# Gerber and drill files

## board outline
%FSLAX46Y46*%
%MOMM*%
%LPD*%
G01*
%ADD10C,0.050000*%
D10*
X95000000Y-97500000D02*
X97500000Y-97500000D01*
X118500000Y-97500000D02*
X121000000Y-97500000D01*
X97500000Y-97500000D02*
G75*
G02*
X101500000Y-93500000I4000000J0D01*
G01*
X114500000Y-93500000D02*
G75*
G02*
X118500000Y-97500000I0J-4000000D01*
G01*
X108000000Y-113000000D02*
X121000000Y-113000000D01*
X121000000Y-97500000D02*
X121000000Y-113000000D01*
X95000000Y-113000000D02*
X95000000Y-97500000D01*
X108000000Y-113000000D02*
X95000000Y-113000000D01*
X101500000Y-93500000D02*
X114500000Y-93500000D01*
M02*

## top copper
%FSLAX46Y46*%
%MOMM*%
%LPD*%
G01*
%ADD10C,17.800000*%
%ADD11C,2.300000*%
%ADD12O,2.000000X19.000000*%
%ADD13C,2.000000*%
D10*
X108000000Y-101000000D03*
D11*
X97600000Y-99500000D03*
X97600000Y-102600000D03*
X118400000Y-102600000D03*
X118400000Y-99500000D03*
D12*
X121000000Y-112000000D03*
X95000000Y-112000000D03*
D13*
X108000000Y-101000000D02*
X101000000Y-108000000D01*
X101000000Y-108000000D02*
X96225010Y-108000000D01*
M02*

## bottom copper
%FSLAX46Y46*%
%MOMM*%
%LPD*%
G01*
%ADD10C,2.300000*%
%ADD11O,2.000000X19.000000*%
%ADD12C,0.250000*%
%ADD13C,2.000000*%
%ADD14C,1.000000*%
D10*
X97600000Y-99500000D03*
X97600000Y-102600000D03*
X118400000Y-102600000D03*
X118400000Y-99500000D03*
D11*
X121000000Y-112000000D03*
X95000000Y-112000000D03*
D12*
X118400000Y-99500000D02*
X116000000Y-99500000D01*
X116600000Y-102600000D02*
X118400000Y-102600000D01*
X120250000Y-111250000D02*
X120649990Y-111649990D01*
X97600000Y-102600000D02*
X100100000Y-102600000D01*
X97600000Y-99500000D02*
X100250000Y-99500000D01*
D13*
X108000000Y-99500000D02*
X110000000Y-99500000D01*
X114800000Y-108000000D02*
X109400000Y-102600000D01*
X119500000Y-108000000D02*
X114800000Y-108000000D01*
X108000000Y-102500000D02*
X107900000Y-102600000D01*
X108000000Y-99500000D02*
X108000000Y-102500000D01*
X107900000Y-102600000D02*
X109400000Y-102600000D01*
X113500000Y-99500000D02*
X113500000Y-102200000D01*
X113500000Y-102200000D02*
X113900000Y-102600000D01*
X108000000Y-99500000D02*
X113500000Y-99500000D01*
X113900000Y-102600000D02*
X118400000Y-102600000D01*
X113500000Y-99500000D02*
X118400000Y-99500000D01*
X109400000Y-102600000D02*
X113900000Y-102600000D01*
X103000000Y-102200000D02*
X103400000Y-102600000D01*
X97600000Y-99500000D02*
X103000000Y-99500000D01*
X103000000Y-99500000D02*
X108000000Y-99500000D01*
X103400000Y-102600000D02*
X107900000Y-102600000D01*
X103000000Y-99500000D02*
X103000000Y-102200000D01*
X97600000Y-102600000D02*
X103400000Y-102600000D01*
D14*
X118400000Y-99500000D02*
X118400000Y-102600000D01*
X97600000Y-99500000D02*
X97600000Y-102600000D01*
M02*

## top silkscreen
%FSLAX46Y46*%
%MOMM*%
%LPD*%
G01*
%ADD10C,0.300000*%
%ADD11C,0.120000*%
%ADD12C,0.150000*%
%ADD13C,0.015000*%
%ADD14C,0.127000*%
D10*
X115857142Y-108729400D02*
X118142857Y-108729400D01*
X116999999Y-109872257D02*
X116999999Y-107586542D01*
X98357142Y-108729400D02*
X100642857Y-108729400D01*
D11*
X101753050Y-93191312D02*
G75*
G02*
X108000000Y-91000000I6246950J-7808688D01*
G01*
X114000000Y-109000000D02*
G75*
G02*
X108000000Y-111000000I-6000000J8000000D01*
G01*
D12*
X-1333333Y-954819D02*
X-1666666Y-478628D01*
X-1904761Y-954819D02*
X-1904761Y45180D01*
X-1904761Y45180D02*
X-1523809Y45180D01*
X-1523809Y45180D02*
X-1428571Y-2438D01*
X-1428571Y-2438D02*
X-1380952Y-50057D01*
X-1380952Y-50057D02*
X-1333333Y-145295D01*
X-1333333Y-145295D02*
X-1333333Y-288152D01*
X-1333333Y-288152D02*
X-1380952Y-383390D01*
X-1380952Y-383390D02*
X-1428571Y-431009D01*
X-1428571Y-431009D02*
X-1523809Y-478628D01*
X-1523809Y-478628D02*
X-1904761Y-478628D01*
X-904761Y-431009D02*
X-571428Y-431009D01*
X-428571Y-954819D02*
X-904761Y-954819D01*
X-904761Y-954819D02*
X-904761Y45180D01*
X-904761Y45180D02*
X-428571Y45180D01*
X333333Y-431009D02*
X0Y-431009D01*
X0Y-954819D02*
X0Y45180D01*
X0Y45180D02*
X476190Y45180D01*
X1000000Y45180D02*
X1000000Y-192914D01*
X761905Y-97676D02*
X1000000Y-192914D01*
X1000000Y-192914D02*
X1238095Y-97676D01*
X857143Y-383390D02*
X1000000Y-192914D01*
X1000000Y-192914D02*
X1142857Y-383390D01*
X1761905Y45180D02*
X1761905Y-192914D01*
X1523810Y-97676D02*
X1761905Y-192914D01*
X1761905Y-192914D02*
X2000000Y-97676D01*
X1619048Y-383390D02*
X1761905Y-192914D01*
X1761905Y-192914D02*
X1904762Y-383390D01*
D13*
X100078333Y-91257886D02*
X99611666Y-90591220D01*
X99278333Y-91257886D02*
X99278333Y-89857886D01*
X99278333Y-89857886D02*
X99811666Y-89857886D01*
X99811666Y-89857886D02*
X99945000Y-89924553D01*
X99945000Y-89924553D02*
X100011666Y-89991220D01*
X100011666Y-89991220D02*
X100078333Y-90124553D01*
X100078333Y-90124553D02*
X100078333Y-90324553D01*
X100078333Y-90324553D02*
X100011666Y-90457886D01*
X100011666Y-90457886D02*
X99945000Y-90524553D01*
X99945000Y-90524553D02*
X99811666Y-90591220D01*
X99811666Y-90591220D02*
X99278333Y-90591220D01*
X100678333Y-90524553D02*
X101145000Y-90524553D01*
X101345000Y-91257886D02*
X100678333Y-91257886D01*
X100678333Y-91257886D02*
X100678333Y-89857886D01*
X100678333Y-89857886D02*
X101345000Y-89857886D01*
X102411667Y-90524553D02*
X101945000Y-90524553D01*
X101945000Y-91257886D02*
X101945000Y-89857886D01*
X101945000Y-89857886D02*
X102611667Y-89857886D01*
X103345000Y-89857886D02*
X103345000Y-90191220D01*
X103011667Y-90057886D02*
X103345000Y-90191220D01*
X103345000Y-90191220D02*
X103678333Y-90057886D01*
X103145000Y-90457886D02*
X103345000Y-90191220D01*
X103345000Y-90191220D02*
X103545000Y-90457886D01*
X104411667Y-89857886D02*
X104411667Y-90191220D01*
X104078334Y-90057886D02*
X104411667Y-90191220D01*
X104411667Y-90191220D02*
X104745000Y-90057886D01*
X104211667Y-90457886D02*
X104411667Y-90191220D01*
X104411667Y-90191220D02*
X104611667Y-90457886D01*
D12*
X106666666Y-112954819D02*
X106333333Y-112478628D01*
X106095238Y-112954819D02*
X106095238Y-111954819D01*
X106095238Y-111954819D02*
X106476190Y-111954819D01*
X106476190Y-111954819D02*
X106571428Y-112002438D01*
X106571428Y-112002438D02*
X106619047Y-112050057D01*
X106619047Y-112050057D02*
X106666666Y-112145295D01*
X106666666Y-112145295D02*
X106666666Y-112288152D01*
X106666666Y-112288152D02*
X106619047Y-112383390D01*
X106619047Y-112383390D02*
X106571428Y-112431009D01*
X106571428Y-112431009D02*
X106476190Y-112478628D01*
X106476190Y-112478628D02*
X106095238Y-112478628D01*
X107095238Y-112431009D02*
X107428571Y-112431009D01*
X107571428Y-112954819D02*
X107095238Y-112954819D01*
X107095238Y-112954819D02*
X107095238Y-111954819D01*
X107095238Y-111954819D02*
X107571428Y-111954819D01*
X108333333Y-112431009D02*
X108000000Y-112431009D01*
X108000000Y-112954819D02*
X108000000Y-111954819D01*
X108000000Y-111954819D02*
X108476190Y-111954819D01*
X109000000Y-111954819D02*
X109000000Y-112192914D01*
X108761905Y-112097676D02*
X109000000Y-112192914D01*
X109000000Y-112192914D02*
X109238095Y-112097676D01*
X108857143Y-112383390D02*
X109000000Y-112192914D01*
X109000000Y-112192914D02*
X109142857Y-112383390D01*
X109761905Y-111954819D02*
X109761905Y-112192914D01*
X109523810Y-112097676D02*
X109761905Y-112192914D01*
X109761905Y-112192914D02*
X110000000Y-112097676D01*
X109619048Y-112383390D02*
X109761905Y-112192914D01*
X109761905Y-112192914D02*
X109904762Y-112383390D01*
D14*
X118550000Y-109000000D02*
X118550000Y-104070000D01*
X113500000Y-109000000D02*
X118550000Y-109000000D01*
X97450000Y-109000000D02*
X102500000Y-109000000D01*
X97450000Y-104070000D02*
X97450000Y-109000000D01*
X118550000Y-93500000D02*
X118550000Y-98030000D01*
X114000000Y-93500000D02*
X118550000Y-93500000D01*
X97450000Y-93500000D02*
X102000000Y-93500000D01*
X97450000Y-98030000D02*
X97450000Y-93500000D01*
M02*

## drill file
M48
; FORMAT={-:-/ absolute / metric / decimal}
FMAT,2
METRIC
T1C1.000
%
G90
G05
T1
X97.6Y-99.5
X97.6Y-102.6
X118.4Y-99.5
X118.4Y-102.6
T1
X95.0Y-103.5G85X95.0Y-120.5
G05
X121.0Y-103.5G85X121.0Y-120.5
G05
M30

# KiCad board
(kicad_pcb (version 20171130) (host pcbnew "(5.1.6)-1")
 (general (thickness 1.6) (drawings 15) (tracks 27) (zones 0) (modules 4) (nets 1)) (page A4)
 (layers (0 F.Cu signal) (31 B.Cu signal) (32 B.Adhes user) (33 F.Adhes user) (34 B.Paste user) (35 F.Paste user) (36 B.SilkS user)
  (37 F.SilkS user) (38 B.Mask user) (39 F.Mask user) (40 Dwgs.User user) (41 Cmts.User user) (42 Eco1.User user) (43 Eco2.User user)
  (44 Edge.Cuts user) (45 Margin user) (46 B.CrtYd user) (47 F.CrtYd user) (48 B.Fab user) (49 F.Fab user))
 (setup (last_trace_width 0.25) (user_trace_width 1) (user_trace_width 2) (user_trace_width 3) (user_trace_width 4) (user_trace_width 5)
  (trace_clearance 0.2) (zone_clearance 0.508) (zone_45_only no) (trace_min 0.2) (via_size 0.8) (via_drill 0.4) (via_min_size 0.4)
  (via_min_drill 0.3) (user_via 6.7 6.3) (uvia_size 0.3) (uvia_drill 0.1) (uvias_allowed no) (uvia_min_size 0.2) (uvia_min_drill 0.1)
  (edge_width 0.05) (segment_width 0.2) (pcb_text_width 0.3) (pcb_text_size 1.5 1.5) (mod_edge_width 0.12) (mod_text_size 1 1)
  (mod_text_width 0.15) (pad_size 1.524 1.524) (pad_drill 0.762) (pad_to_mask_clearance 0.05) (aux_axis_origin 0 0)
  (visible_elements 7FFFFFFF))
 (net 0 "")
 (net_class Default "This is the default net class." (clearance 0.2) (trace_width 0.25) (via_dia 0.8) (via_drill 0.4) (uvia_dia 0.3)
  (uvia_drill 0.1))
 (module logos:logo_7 (layer F.Cu) (at 103.5 101.5)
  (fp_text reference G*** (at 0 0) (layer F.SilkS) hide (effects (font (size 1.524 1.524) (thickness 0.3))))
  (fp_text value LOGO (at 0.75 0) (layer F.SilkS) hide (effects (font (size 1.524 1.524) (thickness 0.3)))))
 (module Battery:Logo (layer F.Cu) (at 0 0)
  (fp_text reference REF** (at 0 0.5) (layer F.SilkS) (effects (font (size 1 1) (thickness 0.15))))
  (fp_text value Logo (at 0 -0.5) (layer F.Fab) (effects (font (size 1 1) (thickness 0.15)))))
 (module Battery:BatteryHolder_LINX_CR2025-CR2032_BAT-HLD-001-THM (layer F.Cu) (at 108 101)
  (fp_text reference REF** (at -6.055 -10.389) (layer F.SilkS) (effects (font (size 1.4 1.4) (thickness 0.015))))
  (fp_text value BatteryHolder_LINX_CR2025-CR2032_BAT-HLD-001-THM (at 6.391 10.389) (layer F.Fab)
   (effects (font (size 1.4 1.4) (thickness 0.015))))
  (fp_line (start 10.55 8) (end 10.55 3.07) (layer F.SilkS) (width 0.127))
  (fp_line (start 5.5 8) (end 10.55 8) (layer F.SilkS) (width 0.127))
  (fp_line (start -10.55 8) (end -5.5 8) (layer F.SilkS) (width 0.127))
  (fp_line (start -10.55 3.07) (end -10.55 8) (layer F.SilkS) (width 0.127))
  (fp_line (start 10.55 -7.5) (end 10.55 -2.97) (layer F.SilkS) (width 0.127))
  (fp_line (start 6 -7.5) (end 10.55 -7.5) (layer F.SilkS) (width 0.127))
  (fp_line (start -10.55 -7.5) (end -6 -7.5) (layer F.SilkS) (width 0.127))
  (fp_line (start -10.55 -2.97) (end -10.55 -7.5) (layer F.SilkS) (width 0.127))
  (pad N smd circle (at 0 0) (size 17.8 17.8) (layers F.Cu F.Mask))
  (pad P1 thru_hole circle (at -10.4 -1.5) (size 2.3 2.3) (drill 1) (layers *.Cu *.Mask))
  (pad P2 thru_hole circle (at -10.4 1.6) (size 2.3 2.3) (drill 1) (layers *.Cu *.Mask))
  (pad P3 thru_hole circle (at 10.4 1.6) (size 2.3 2.3) (drill 1) (layers *.Cu *.Mask))
  (pad P4 thru_hole circle (at 10.4 -1.5) (size 2.3 2.3) (drill 1) (layers *.Cu *.Mask)))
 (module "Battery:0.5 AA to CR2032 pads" (layer F.Cu) (at 108 112)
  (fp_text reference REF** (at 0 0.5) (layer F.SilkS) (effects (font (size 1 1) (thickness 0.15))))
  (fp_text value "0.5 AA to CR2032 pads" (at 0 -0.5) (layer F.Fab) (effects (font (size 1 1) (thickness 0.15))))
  (pad 2 thru_hole oval (at 13 0) (size 2 19) (drill oval 1 18) (layers *.Cu *.Mask))
  (pad 1 thru_hole oval (at -13 0) (size 2 19) (drill oval 1 18) (layers *.Cu *.Mask)))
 (gr_line (start 95 97.5) (end 97.5 97.5) (layer Edge.Cuts) (width 0.05))
 (gr_line (start 118.5 97.5) (end 121 97.5) (layer Edge.Cuts) (width 0.05))
 (gr_arc (start 101.5 97.5) (end 101.5 93.5) (angle -90) (layer Edge.Cuts) (width 0.05))
 (gr_arc (start 114.5 97.5) (end 118.5 97.5) (angle -90) (layer Edge.Cuts) (width 0.05))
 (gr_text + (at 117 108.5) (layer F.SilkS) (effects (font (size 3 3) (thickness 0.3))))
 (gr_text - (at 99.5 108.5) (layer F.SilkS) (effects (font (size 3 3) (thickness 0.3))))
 (gr_line (start 108 113) (end 121 113) (layer Edge.Cuts) (width 0.05))
 (gr_line (start 121 97.5) (end 121 113) (layer Edge.Cuts) (width 0.05))
 (gr_line (start 95 113) (end 95 97.5) (layer Edge.Cuts) (width 0.05))
 (gr_line (start 108 113) (end 95 113) (layer Edge.Cuts) (width 0.05))
 (gr_line (start 101.5 93.5) (end 114.5 93.5) (layer Edge.Cuts) (width 0.05))
 (gr_arc (start 108 101) (end 108 91) (angle -38.65980825) (layer F.SilkS) (width 0.12))
 (gr_arc (start 108 101) (end 108 111) (angle -36.86989765) (layer F.SilkS) (width 0.12))
 (segment (start 118.4 99.5) (end 116 99.5) (width 0.25) (layer B.Cu) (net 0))
 (segment (start 116.6 102.6) (end 118.4 102.6) (width 0.25) (layer B.Cu) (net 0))
 (segment (start 120.25 111.25) (end 120.64999 111.64999) (width 0.25) (layer B.Cu) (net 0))
 (segment (start 97.6 102.6) (end 100.1 102.6) (width 0.25) (layer B.Cu) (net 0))
 (segment (start 97.6 99.5) (end 100.25 99.5) (width 0.25) (layer B.Cu) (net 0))
 (segment (start 108 101) (end 101 108) (width 2) (layer F.Cu) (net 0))
 (segment (start 101 108) (end 96.22501 108) (width 2) (layer F.Cu) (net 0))
 (segment (start 108 99.5) (end 110 99.5) (width 2) (layer B.Cu) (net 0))
 (segment (start 114.8 108) (end 109.4 102.6) (width 2) (layer B.Cu) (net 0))
 (segment (start 119.5 108) (end 114.8 108) (width 2) (layer B.Cu) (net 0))
 (segment (start 108 102.5) (end 107.9 102.6) (width 2) (layer B.Cu) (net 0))
 (segment (start 108 99.5) (end 108 102.5) (width 2) (layer B.Cu) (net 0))
 (segment (start 107.9 102.6) (end 109.4 102.6) (width 2) (layer B.Cu) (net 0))
 (segment (start 113.5 99.5) (end 113.5 102.2) (width 2) (layer B.Cu) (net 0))
 (segment (start 113.5 102.2) (end 113.9 102.6) (width 2) (layer B.Cu) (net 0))
 (segment (start 108 99.5) (end 113.5 99.5) (width 2) (layer B.Cu) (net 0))
 (segment (start 113.9 102.6) (end 118.4 102.6) (width 2) (layer B.Cu) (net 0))
 (segment (start 113.5 99.5) (end 118.4 99.5) (width 2) (layer B.Cu) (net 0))
 (segment (start 109.4 102.6) (end 113.9 102.6) (width 2) (layer B.Cu) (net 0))
 (segment (start 103 102.2) (end 103.4 102.6) (width 2) (layer B.Cu) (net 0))
 (segment (start 97.6 99.5) (end 103 99.5) (width 2) (layer B.Cu) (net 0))
 (segment (start 103 99.5) (end 108 99.5) (width 2) (layer B.Cu) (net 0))
 (segment (start 103.4 102.6) (end 107.9 102.6) (width 2) (layer B.Cu) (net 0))
 (segment (start 103 99.5) (end 103 102.2) (width 2) (layer B.Cu) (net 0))
 (segment (start 97.6 102.6) (end 103.4 102.6) (width 2) (layer B.Cu) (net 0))
 (segment (start 118.4 99.5) (end 118.4 102.6) (width 1) (layer B.Cu) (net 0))
 (segment (start 97.6 99.5) (end 97.6 102.6) (width 1) (layer B.Cu) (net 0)))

